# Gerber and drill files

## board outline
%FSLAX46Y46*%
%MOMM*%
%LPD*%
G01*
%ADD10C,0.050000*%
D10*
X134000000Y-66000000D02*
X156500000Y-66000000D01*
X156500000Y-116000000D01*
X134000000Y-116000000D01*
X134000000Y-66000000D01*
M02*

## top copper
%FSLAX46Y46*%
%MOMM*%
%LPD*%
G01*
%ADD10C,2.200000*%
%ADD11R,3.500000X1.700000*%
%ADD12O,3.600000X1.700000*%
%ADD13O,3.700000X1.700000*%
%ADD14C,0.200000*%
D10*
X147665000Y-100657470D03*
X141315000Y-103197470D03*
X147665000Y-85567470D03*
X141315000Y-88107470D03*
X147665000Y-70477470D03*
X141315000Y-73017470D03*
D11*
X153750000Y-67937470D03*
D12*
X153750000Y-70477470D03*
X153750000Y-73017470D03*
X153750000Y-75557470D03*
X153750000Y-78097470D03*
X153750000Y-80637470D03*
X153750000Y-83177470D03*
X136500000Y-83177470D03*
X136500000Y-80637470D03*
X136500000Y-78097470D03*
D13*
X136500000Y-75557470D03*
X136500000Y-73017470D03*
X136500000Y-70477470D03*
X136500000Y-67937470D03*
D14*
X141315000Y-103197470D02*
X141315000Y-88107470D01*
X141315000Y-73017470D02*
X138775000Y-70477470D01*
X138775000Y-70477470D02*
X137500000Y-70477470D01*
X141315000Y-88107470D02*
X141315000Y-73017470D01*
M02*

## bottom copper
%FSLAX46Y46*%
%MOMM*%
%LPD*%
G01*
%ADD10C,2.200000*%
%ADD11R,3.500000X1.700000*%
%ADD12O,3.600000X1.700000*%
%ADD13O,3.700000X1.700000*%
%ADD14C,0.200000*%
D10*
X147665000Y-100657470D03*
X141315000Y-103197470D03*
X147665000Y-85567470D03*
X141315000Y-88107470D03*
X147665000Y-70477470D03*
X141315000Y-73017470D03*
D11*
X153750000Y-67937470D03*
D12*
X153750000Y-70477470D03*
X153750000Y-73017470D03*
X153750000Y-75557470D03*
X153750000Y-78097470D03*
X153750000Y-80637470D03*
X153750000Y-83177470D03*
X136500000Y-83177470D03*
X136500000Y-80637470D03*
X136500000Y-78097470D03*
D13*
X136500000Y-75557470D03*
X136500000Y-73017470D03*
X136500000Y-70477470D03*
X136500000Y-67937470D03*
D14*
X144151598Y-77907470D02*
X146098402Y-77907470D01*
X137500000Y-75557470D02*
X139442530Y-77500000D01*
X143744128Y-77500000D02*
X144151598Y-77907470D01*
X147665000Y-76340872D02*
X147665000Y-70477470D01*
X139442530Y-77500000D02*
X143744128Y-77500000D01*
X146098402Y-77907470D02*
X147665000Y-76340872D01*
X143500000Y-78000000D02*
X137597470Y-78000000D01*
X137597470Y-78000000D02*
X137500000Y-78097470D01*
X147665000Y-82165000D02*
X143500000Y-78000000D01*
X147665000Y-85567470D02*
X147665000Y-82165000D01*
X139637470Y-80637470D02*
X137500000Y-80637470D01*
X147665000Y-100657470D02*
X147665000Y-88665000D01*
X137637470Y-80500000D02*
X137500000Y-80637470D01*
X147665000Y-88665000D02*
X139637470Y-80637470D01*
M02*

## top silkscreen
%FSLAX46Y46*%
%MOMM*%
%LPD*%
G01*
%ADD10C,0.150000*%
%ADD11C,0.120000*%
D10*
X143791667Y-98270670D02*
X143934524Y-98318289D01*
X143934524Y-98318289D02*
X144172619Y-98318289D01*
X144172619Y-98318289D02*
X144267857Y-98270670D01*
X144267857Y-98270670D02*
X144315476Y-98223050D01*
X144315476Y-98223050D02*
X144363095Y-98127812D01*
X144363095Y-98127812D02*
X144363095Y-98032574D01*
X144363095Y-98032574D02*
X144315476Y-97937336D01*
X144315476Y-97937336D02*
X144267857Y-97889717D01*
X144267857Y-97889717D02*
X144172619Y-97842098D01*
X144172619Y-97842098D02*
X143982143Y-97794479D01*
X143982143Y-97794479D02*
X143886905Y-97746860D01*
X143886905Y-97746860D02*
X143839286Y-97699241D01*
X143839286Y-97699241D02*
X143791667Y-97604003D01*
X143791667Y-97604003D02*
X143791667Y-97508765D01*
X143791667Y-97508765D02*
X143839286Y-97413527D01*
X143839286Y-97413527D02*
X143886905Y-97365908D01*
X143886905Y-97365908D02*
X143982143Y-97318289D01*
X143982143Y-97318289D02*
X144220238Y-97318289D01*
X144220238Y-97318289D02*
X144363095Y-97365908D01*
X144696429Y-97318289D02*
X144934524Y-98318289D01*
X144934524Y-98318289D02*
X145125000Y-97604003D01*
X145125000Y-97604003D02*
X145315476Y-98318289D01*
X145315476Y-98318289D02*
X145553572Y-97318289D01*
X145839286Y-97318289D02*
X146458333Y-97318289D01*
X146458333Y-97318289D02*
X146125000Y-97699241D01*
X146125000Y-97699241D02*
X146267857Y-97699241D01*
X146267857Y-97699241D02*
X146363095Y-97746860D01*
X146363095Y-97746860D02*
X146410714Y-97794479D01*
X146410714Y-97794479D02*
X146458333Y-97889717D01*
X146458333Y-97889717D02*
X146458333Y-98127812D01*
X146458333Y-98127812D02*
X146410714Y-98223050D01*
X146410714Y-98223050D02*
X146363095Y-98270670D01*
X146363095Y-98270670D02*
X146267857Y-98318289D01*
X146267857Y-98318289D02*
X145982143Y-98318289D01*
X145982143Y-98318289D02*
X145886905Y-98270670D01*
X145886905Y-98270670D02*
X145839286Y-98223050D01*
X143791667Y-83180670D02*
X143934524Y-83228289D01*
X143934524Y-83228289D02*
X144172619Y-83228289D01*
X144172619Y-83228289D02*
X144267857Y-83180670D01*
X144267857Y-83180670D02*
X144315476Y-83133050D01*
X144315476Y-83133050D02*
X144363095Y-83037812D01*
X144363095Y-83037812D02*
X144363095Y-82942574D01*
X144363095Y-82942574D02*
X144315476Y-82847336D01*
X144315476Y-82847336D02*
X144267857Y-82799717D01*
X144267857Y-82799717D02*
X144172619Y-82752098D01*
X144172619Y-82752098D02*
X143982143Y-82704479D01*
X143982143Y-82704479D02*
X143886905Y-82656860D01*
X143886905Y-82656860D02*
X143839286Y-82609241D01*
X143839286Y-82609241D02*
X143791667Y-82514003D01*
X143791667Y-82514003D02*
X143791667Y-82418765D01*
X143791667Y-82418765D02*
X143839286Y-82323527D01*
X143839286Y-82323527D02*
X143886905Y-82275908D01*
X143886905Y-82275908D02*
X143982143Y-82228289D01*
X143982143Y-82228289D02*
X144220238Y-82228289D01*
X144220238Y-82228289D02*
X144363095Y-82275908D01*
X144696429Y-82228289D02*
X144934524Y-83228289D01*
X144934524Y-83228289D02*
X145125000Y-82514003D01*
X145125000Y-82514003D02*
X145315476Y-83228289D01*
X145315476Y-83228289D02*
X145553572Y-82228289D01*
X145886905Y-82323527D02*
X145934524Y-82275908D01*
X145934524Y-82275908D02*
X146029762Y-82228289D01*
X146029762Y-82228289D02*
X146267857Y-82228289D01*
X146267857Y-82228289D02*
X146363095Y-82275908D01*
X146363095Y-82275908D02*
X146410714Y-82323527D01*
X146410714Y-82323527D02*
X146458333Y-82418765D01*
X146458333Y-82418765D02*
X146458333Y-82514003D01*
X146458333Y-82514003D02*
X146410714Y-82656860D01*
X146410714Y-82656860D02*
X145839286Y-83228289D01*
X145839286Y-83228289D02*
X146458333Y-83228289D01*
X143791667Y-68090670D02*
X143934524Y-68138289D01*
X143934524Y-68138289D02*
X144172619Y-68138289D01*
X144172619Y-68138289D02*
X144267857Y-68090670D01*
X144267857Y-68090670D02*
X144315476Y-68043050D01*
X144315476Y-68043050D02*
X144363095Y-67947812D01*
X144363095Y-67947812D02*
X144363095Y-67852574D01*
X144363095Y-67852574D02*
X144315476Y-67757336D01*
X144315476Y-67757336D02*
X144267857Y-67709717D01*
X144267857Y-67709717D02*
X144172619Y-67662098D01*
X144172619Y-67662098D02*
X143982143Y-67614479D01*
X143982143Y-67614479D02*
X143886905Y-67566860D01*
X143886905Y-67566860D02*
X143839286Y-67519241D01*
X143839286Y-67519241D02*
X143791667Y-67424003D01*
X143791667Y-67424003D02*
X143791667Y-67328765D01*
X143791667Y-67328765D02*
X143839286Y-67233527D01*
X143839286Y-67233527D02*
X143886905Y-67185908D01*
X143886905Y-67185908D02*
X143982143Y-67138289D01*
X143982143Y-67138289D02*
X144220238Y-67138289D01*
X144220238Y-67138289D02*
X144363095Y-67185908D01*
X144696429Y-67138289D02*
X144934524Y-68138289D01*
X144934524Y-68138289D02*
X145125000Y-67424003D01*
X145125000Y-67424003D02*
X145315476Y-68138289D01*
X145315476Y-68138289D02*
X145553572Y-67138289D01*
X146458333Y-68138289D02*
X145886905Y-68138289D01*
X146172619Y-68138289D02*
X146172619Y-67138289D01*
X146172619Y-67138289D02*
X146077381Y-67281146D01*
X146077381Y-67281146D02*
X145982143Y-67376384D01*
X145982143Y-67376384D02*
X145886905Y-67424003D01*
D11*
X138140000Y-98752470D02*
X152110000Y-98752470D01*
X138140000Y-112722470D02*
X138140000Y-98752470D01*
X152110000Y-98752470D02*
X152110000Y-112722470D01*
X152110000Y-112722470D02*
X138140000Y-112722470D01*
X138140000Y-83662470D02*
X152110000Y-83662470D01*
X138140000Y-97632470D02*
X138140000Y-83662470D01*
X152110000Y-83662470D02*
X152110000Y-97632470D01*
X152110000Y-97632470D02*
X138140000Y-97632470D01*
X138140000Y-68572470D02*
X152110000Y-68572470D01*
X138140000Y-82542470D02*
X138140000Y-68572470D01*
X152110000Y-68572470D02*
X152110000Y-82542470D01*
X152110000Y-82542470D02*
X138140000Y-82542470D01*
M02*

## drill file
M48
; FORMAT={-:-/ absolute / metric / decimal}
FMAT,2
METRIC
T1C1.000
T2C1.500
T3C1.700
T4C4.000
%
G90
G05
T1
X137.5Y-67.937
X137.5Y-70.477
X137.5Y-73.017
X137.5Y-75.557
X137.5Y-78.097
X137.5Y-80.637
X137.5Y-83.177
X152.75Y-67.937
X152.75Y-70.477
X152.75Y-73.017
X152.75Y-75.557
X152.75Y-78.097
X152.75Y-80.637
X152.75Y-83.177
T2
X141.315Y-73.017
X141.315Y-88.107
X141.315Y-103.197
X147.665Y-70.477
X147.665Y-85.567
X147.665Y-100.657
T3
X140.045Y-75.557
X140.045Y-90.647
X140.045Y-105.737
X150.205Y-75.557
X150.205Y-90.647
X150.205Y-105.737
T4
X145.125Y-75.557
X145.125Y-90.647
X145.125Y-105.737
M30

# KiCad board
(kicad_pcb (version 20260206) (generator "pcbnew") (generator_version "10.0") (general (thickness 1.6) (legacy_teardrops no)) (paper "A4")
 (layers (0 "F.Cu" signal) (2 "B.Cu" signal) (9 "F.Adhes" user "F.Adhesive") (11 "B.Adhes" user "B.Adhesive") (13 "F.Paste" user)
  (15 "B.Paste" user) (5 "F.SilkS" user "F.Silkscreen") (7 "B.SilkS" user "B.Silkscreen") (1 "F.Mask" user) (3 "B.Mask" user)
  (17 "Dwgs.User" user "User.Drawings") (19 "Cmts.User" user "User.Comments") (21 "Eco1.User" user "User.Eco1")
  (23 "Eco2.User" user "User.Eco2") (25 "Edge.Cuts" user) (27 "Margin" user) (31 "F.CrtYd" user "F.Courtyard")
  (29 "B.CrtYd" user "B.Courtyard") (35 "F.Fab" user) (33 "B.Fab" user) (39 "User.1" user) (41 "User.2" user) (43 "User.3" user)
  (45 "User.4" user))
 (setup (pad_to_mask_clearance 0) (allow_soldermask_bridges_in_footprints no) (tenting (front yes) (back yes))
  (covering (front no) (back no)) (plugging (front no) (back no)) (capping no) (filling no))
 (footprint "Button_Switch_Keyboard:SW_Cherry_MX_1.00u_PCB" (layer "F.Cu") (at 147.665 100.65747)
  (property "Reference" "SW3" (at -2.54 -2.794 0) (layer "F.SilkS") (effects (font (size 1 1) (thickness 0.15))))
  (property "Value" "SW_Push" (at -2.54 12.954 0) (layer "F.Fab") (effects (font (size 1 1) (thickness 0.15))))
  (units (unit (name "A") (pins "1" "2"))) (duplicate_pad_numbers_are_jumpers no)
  (fp_line (start -9.525 -1.905) (end 4.445 -1.905) (stroke (width 0.12) (type solid)) (layer "F.SilkS"))
  (fp_line (start -9.525 12.065) (end -9.525 -1.905) (stroke (width 0.12) (type solid)) (layer "F.SilkS"))
  (fp_line (start 4.445 -1.905) (end 4.445 12.065) (stroke (width 0.12) (type solid)) (layer "F.SilkS"))
  (fp_line (start 4.445 12.065) (end -9.525 12.065) (stroke (width 0.12) (type solid)) (layer "F.SilkS"))
  (pad "" np_thru_hole circle (at -7.62 5.08) (size 1.7 1.7) (drill 1.7) (layers "*.Cu" "*.Mask"))
  (pad "" np_thru_hole circle (at -2.54 5.08) (size 4 4) (drill 4) (layers "*.Cu" "*.Mask"))
  (pad "" np_thru_hole circle (at 2.54 5.08) (size 1.7 1.7) (drill 1.7) (layers "*.Cu" "*.Mask"))
  (pad "1" thru_hole circle (at 0 0) (size 2.2 2.2) (drill 1.5) (layers "*.Cu" "*.Mask") (remove_unused_layers no)
   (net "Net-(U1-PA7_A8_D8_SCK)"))
  (pad "2" thru_hole circle (at -6.35 2.54) (size 2.2 2.2) (drill 1.5) (layers "*.Cu" "*.Mask") (remove_unused_layers no) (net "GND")))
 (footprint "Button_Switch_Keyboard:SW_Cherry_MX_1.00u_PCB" (layer "F.Cu") (at 147.665 85.56747)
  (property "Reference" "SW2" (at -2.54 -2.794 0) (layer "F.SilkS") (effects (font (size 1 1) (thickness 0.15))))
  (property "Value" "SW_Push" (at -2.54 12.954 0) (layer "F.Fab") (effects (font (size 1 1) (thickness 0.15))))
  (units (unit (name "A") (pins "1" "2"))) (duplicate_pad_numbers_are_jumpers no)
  (fp_line (start -9.525 -1.905) (end 4.445 -1.905) (stroke (width 0.12) (type solid)) (layer "F.SilkS"))
  (fp_line (start -9.525 12.065) (end -9.525 -1.905) (stroke (width 0.12) (type solid)) (layer "F.SilkS"))
  (fp_line (start 4.445 -1.905) (end 4.445 12.065) (stroke (width 0.12) (type solid)) (layer "F.SilkS"))
  (fp_line (start 4.445 12.065) (end -9.525 12.065) (stroke (width 0.12) (type solid)) (layer "F.SilkS"))
  (pad "" np_thru_hole circle (at -7.62 5.08) (size 1.7 1.7) (drill 1.7) (layers "*.Cu" "*.Mask"))
  (pad "" np_thru_hole circle (at -2.54 5.08) (size 4 4) (drill 4) (layers "*.Cu" "*.Mask"))
  (pad "" np_thru_hole circle (at 2.54 5.08) (size 1.7 1.7) (drill 1.7) (layers "*.Cu" "*.Mask"))
  (pad "1" thru_hole circle (at 0 0) (size 2.2 2.2) (drill 1.5) (layers "*.Cu" "*.Mask") (remove_unused_layers no)
   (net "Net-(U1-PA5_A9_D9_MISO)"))
  (pad "2" thru_hole circle (at -6.35 2.54) (size 2.2 2.2) (drill 1.5) (layers "*.Cu" "*.Mask") (remove_unused_layers no) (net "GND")))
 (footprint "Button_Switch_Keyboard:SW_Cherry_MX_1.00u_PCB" (layer "F.Cu") (at 147.665 70.47747)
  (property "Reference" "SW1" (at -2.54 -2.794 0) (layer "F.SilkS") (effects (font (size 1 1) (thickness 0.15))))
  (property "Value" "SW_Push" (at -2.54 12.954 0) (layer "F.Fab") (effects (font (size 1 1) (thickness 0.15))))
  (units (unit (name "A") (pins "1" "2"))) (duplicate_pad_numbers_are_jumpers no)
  (fp_line (start -9.525 -1.905) (end 4.445 -1.905) (stroke (width 0.12) (type solid)) (layer "F.SilkS"))
  (fp_line (start -9.525 12.065) (end -9.525 -1.905) (stroke (width 0.12) (type solid)) (layer "F.SilkS"))
  (fp_line (start 4.445 -1.905) (end 4.445 12.065) (stroke (width 0.12) (type solid)) (layer "F.SilkS"))
  (fp_line (start 4.445 12.065) (end -9.525 12.065) (stroke (width 0.12) (type solid)) (layer "F.SilkS"))
  (pad "" np_thru_hole circle (at -7.62 5.08) (size 1.7 1.7) (drill 1.7) (layers "*.Cu" "*.Mask"))
  (pad "" np_thru_hole circle (at -2.54 5.08) (size 4 4) (drill 4) (layers "*.Cu" "*.Mask"))
  (pad "" np_thru_hole circle (at 2.54 5.08) (size 1.7 1.7) (drill 1.7) (layers "*.Cu" "*.Mask"))
  (pad "1" thru_hole circle (at 0 0) (size 2.2 2.2) (drill 1.5) (layers "*.Cu" "*.Mask") (remove_unused_layers no)
   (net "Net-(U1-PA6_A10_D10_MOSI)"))
  (pad "2" thru_hole circle (at -6.35 2.54) (size 2.2 2.2) (drill 1.5) (layers "*.Cu" "*.Mask") (remove_unused_layers no) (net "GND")))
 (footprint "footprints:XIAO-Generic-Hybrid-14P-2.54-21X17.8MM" (layer "B.Cu") (at 145.125 75.55747 180)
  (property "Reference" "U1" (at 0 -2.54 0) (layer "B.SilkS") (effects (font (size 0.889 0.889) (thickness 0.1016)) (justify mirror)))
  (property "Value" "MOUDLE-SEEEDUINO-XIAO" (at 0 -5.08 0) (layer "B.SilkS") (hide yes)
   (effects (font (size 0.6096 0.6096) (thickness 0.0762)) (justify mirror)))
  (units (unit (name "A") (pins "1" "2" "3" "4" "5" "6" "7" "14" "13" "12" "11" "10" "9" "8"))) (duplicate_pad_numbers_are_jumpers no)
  (pad "1" thru_hole rect (at -7.625 7.62 180) (size 3.5 1.7) (drill 1 (offset -1 0)) (layers "*.Cu" "*.Mask") (remove_unused_layers no)
   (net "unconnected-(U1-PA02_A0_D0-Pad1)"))
  (pad "2" thru_hole oval (at -7.625 5.08 180) (size 3.6 1.7) (drill 1 (offset -1 0)) (layers "*.Cu" "*.Mask") (remove_unused_layers no)
   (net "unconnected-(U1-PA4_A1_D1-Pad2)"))
  (pad "3" thru_hole oval (at -7.625 2.54 180) (size 3.6 1.7) (drill 1 (offset -1 0)) (layers "*.Cu" "*.Mask") (remove_unused_layers no)
   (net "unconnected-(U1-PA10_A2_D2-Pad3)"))
  (pad "4" thru_hole oval (at -7.625 0 180) (size 3.6 1.7) (drill 1 (offset -1 0)) (layers "*.Cu" "*.Mask") (remove_unused_layers no)
   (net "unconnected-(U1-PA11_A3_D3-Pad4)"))
  (pad "5" thru_hole oval (at -7.625 -2.54 180) (size 3.6 1.7) (drill 1 (offset -1 0)) (layers "*.Cu" "*.Mask") (remove_unused_layers no)
   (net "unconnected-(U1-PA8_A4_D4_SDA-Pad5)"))
  (pad "6" thru_hole oval (at -7.625 -5.08) (size 3.6 1.7) (drill 1 (offset 1 0)) (layers "*.Cu" "*.Mask") (remove_unused_layers no)
   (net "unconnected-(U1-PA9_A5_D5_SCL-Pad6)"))
  (pad "7" thru_hole oval (at -7.625 -7.62 180) (size 3.6 1.7) (drill 1 (offset -1 0)) (layers "*.Cu" "*.Mask") (remove_unused_layers no)
   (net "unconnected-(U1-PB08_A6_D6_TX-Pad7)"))
  (pad "8" thru_hole oval (at 7.625 -7.62 180) (size 3.6 1.7) (drill 1 (offset 1 0)) (layers "*.Cu" "*.Mask") (remove_unused_layers no)
   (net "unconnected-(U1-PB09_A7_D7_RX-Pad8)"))
  (pad "9" thru_hole oval (at 7.625 -5.08 180) (size 3.6 1.7) (drill 1 (offset 1 0)) (layers "*.Cu" "*.Mask") (remove_unused_layers no)
   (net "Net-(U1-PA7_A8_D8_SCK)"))
  (pad "10" thru_hole oval (at 7.625 -2.54 180) (size 3.6 1.7) (drill 1 (offset 1 0)) (layers "*.Cu" "*.Mask") (remove_unused_layers no)
   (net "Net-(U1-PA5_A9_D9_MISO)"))
  (pad "11" thru_hole oval (at 7.625 0 180) (size 3.7 1.7) (drill 1 (offset 1 0)) (layers "*.Cu" "*.Mask") (remove_unused_layers no)
   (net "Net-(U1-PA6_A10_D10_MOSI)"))
  (pad "12" thru_hole oval (at 7.625 2.54 180) (size 3.7 1.7) (drill 1 (offset 1 0)) (layers "*.Cu" "*.Mask") (remove_unused_layers no)
   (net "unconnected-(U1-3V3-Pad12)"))
  (pad "13" thru_hole oval (at 7.625 5.08 180) (size 3.7 1.7) (drill 1 (offset 1 0)) (layers "*.Cu" "*.Mask") (remove_unused_layers no)
   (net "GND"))
  (pad "14" thru_hole oval (at 7.625 7.62 180) (size 3.7 1.7) (drill 1 (offset 1 0)) (layers "*.Cu" "*.Mask") (remove_unused_layers no)
   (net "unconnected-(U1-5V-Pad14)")))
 (gr_rect (start 134 66) (end 156.5 116) (stroke (width 0.05) (type default)) (fill no) (layer "Edge.Cuts"))
 (segment (start 141.315 103.19747) (end 141.315 88.10747) (width 0.2) (layer "F.Cu") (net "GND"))
 (segment (start 141.315 73.01747) (end 138.775 70.47747) (width 0.2) (layer "F.Cu") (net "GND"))
 (segment (start 138.775 70.47747) (end 137.5 70.47747) (width 0.2) (layer "F.Cu") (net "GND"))
 (segment (start 141.315 88.10747) (end 141.315 73.01747) (width 0.2) (layer "F.Cu") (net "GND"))
 (segment (start 144.151598 77.90747) (end 146.098402 77.90747) (width 0.2) (layer "B.Cu") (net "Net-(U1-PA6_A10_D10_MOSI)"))
 (segment (start 137.5 75.55747) (end 139.44253 77.5) (width 0.2) (layer "B.Cu") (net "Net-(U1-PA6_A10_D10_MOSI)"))
 (segment (start 143.744128 77.5) (end 144.151598 77.90747) (width 0.2) (layer "B.Cu") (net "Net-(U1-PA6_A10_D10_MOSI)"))
 (segment (start 147.665 76.340872) (end 147.665 70.47747) (width 0.2) (layer "B.Cu") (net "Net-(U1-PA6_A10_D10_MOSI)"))
 (segment (start 139.44253 77.5) (end 143.744128 77.5) (width 0.2) (layer "B.Cu") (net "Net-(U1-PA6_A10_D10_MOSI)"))
 (segment (start 146.098402 77.90747) (end 147.665 76.340872) (width 0.2) (layer "B.Cu") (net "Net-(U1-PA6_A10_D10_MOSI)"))
 (segment (start 143.5 78) (end 137.59747 78) (width 0.2) (layer "B.Cu") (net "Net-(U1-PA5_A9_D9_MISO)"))
 (segment (start 137.59747 78) (end 137.5 78.09747) (width 0.2) (layer "B.Cu") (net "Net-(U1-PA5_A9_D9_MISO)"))
 (segment (start 147.665 82.165) (end 143.5 78) (width 0.2) (layer "B.Cu") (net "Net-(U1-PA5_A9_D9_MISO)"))
 (segment (start 147.665 85.56747) (end 147.665 82.165) (width 0.2) (layer "B.Cu") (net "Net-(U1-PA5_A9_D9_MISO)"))
 (segment (start 139.63747 80.63747) (end 137.5 80.63747) (width 0.2) (layer "B.Cu") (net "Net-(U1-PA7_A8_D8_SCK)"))
 (segment (start 147.665 100.65747) (end 147.665 88.665) (width 0.2) (layer "B.Cu") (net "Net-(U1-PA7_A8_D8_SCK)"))
 (segment (start 137.63747 80.5) (end 137.5 80.63747) (width 0.2) (layer "B.Cu") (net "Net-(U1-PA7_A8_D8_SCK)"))
 (segment (start 147.665 88.665) (end 139.63747 80.63747) (width 0.2) (layer "B.Cu") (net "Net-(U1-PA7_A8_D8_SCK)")))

